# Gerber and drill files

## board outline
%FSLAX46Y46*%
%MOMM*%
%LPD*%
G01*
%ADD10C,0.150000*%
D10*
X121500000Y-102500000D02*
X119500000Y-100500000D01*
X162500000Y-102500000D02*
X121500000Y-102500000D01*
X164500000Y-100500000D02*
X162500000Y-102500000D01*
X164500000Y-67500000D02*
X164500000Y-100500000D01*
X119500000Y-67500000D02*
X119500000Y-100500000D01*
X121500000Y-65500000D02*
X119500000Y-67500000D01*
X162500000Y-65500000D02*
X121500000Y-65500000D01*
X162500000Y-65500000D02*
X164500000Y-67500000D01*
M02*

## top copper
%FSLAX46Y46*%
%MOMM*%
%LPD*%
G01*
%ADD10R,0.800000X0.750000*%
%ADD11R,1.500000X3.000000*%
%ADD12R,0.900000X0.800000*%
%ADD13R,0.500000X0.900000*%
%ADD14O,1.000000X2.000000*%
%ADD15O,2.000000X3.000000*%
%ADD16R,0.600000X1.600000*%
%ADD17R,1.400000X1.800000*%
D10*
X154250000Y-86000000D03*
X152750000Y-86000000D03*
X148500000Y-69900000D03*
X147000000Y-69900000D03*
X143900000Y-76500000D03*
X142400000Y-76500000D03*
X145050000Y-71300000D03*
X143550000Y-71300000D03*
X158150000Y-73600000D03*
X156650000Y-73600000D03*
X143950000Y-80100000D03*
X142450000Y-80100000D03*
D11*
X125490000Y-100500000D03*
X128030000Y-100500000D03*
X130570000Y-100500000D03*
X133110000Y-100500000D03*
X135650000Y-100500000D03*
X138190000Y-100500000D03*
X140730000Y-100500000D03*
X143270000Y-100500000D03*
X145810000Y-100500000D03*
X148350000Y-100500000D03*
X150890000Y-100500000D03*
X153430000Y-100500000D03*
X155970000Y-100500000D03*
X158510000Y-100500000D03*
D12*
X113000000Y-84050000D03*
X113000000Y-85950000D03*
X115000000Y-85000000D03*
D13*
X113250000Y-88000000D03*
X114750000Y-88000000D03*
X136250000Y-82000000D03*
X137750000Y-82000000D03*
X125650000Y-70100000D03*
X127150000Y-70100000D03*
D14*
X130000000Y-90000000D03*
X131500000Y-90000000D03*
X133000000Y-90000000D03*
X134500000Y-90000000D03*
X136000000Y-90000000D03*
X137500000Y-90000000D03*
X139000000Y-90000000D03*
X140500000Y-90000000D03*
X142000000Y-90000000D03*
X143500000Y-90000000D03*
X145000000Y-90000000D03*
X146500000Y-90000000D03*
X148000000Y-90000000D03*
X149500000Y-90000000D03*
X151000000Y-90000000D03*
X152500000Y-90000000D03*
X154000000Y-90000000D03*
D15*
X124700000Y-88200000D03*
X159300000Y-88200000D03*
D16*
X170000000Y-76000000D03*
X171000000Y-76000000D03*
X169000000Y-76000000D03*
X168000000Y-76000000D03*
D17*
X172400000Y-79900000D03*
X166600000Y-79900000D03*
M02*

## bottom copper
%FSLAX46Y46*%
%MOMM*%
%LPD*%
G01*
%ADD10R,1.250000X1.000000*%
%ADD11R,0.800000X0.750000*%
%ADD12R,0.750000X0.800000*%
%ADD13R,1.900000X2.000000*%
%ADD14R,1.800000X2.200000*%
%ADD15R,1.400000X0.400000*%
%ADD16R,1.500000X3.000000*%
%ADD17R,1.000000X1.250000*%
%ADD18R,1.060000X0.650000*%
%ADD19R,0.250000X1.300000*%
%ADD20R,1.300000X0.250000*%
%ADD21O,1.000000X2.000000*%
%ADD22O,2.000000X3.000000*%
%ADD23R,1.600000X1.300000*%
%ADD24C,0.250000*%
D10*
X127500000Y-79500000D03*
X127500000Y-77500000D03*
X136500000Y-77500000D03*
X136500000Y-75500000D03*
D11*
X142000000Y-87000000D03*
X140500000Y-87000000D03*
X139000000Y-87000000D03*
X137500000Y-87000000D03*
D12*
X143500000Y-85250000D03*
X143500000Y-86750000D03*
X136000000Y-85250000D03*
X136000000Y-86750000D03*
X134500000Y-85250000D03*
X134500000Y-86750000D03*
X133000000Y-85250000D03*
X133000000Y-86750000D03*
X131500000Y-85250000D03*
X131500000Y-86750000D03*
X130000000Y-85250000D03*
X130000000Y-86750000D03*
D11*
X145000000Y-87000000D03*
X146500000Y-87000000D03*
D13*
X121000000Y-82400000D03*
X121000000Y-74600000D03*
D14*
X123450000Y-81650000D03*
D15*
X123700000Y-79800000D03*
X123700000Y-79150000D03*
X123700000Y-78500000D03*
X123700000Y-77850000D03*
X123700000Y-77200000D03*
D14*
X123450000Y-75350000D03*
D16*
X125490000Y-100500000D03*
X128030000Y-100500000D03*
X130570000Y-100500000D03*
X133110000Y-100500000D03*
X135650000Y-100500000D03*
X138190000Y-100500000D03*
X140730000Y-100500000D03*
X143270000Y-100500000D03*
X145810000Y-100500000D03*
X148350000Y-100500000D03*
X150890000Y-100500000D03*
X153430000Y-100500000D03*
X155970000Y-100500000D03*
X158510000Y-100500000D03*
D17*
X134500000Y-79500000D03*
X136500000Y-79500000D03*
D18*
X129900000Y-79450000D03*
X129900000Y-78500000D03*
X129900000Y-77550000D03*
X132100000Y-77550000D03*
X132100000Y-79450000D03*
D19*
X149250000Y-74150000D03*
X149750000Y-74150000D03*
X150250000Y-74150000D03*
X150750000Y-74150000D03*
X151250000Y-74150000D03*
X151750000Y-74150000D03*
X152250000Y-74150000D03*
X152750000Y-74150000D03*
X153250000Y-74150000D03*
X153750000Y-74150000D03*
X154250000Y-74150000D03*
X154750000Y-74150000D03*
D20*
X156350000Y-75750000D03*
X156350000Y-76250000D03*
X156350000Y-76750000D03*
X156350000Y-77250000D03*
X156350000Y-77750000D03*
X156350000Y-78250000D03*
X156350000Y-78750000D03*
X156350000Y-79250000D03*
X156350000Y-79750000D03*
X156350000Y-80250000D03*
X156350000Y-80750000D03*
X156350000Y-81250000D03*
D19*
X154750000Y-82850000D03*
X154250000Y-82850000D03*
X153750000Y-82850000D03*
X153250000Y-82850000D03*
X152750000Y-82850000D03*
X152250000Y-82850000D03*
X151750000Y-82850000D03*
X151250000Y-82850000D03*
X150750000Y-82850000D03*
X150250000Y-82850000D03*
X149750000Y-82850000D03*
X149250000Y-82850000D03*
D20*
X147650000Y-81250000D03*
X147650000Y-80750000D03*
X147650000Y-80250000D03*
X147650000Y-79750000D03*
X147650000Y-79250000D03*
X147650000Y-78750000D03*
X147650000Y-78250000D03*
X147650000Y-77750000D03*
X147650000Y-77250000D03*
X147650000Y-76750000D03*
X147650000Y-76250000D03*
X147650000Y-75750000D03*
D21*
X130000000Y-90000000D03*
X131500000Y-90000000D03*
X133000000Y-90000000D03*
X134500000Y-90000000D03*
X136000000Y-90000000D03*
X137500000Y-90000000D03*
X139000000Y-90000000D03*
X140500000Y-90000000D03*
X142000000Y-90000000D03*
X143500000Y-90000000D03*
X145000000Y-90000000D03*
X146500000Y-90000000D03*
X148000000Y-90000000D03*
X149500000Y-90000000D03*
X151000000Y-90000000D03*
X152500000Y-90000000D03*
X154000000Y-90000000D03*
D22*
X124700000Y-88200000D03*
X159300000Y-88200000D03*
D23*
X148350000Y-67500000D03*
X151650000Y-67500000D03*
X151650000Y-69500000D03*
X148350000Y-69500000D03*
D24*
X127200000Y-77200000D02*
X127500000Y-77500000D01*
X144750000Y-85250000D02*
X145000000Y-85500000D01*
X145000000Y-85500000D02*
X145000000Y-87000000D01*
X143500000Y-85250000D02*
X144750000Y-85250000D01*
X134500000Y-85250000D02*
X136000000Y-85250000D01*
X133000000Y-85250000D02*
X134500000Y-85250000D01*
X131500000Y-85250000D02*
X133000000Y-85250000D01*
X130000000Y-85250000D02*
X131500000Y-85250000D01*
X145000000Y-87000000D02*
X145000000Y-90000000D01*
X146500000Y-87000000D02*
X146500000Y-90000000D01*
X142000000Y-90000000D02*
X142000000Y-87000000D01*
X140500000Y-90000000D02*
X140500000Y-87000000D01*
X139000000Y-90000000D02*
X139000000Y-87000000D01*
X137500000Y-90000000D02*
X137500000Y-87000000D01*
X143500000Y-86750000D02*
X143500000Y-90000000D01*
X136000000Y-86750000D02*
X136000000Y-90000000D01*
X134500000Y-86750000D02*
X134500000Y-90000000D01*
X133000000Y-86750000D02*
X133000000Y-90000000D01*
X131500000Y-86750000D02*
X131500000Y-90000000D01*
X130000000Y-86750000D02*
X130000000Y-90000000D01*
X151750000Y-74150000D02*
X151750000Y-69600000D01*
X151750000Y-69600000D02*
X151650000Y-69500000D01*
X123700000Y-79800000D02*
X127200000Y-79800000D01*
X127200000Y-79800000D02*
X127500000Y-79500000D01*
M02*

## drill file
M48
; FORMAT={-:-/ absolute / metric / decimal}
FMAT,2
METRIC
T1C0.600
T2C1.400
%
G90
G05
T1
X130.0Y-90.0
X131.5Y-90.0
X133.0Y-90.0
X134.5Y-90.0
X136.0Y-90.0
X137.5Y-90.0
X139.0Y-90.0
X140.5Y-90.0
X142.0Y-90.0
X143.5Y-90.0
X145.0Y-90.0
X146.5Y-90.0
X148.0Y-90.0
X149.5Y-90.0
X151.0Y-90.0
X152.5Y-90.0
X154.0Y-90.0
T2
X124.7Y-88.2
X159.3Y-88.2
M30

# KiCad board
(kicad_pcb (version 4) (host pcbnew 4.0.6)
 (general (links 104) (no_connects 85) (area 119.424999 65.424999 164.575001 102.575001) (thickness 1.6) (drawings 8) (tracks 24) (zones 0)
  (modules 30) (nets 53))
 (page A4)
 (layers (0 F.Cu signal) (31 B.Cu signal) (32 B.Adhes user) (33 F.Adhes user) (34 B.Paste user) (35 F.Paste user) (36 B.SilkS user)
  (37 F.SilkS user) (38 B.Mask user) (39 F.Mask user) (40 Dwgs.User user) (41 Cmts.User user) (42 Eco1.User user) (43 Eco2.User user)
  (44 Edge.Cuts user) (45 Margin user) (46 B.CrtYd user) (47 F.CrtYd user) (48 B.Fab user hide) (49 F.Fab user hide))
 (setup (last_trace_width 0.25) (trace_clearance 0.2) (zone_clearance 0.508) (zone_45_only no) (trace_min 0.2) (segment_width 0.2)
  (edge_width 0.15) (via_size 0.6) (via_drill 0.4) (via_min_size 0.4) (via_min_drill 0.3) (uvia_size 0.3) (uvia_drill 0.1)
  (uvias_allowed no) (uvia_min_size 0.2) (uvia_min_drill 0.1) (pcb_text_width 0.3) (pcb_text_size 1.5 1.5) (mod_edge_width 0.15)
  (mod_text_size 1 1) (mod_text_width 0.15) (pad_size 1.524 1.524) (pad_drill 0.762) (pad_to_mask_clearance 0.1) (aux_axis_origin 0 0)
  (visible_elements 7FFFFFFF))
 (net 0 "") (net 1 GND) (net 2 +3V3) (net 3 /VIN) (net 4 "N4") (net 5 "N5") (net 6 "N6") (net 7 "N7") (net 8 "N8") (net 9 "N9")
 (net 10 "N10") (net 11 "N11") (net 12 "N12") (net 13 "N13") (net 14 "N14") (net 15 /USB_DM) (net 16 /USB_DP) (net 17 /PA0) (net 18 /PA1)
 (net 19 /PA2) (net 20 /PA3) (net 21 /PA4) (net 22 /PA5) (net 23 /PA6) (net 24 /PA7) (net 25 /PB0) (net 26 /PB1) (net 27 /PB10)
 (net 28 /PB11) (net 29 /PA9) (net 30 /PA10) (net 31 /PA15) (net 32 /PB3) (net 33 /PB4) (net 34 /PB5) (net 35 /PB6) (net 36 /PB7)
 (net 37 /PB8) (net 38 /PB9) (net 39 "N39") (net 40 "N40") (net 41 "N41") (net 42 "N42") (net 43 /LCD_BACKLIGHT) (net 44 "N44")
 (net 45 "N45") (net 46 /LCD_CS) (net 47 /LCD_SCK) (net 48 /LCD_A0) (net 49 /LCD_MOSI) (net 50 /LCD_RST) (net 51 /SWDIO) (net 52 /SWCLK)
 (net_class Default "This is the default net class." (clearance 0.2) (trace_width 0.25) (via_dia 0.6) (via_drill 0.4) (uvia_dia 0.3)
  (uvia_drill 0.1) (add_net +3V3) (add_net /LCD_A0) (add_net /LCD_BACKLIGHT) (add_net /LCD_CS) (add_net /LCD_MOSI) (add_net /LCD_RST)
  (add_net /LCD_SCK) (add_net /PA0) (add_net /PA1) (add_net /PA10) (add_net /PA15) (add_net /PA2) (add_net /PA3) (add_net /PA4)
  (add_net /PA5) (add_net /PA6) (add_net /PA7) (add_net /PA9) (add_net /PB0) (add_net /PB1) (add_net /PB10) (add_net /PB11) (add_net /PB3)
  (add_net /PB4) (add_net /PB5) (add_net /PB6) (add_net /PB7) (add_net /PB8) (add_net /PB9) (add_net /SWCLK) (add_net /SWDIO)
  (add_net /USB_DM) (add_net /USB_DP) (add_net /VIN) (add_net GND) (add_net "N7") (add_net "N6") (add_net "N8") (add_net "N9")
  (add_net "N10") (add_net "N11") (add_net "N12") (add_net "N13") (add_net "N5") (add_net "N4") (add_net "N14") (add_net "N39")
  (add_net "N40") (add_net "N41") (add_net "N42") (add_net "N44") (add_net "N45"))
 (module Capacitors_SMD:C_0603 (layer F.Cu) (at 153.5 86)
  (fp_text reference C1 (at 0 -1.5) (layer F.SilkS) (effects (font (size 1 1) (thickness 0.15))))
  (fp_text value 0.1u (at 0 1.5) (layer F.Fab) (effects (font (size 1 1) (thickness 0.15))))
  (pad 2 smd rect (at 0.75 0) (size 0.8 0.75) (layers F.Cu F.Paste F.Mask) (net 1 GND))
  (pad 1 smd rect (at -0.75 0) (size 0.8 0.75) (layers F.Cu F.Paste F.Mask) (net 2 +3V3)))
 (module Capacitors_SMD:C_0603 (layer F.Cu) (at 147.75 69.9)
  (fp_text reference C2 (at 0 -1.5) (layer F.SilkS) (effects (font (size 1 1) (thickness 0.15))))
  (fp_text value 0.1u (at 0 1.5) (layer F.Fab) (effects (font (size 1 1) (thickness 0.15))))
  (pad 2 smd rect (at 0.75 0) (size 0.8 0.75) (layers F.Cu F.Paste F.Mask) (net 1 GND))
  (pad 1 smd rect (at -0.75 0) (size 0.8 0.75) (layers F.Cu F.Paste F.Mask) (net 2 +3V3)))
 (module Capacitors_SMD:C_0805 (layer B.Cu) (at 127.5 78.5 90)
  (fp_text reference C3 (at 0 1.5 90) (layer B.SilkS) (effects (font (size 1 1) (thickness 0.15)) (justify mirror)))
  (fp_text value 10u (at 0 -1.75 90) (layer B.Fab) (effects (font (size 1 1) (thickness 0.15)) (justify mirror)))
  (pad 1 smd rect (at -1 0 90) (size 1 1.25) (layers B.Cu B.Paste B.Mask) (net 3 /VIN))
  (pad 2 smd rect (at 1 0 90) (size 1 1.25) (layers B.Cu B.Paste B.Mask) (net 1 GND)))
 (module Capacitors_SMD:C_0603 (layer F.Cu) (at 143.15 76.5)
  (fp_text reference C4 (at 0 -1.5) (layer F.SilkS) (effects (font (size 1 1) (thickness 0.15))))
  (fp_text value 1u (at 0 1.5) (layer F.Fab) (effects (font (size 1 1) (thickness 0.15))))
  (pad 2 smd rect (at 0.75 0) (size 0.8 0.75) (layers F.Cu F.Paste F.Mask) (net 2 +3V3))
  (pad 1 smd rect (at -0.75 0) (size 0.8 0.75) (layers F.Cu F.Paste F.Mask) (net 1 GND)))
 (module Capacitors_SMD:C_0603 (layer F.Cu) (at 144.3 71.3)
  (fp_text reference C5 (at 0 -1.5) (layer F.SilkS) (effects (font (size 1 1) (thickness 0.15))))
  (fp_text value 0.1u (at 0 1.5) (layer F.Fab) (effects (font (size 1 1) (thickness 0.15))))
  (pad 2 smd rect (at 0.75 0) (size 0.8 0.75) (layers F.Cu F.Paste F.Mask) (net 1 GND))
  (pad 1 smd rect (at -0.75 0) (size 0.8 0.75) (layers F.Cu F.Paste F.Mask) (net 2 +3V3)))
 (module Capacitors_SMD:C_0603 (layer F.Cu) (at 157.4 73.6)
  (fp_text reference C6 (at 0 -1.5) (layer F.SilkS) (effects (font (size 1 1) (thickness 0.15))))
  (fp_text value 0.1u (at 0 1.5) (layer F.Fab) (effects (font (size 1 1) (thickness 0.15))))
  (pad 2 smd rect (at 0.75 0) (size 0.8 0.75) (layers F.Cu F.Paste F.Mask) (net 1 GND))
  (pad 1 smd rect (at -0.75 0) (size 0.8 0.75) (layers F.Cu F.Paste F.Mask) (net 2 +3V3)))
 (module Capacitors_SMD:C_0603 (layer F.Cu) (at 143.2 80.1)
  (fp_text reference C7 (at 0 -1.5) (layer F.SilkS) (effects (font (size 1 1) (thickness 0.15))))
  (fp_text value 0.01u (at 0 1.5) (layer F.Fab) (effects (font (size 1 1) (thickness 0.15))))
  (pad 2 smd rect (at 0.75 0) (size 0.8 0.75) (layers F.Cu F.Paste F.Mask) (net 2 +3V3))
  (pad 1 smd rect (at -0.75 0) (size 0.8 0.75) (layers F.Cu F.Paste F.Mask) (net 1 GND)))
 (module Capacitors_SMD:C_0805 (layer B.Cu) (at 136.5 76.5 90)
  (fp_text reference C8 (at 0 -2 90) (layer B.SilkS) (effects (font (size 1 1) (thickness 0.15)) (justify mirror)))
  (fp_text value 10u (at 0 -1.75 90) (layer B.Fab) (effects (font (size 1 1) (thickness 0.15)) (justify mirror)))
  (pad 1 smd rect (at -1 0 90) (size 1 1.25) (layers B.Cu B.Paste B.Mask) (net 2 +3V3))
  (pad 2 smd rect (at 1 0 90) (size 1 1.25) (layers B.Cu B.Paste B.Mask) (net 1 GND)))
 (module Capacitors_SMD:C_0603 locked (layer B.Cu) (at 141.25 87)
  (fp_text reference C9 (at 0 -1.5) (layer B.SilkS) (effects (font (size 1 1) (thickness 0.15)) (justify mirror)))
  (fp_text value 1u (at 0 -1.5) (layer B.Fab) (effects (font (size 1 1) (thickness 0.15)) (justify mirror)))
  (pad 2 smd rect (at 0.75 0) (size 0.8 0.75) (layers B.Cu B.Paste B.Mask) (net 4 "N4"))
  (pad 1 smd rect (at -0.75 0) (size 0.8 0.75) (layers B.Cu B.Paste B.Mask) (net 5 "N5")))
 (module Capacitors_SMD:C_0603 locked (layer B.Cu) (at 138.25 87)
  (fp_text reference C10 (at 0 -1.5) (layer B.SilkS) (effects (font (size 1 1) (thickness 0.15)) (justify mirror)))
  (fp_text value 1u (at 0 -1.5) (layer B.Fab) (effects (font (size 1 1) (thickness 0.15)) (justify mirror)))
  (pad 2 smd rect (at 0.75 0) (size 0.8 0.75) (layers B.Cu B.Paste B.Mask) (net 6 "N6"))
  (pad 1 smd rect (at -0.75 0) (size 0.8 0.75) (layers B.Cu B.Paste B.Mask) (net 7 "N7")))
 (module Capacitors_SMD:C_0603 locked (layer B.Cu) (at 143.5 86 90)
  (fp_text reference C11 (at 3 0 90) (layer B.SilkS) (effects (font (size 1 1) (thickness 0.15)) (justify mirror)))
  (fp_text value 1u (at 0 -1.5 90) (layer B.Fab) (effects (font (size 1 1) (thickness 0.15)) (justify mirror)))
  (pad 2 smd rect (at 0.75 0 90) (size 0.8 0.75) (layers B.Cu B.Paste B.Mask) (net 1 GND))
  (pad 1 smd rect (at -0.75 0 90) (size 0.8 0.75) (layers B.Cu B.Paste B.Mask) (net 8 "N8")))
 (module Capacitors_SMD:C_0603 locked (layer B.Cu) (at 136 86 90)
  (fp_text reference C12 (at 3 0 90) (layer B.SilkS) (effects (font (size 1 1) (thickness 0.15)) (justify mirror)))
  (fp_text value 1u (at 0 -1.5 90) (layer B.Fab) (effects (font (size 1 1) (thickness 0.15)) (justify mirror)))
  (pad 2 smd rect (at 0.75 0 90) (size 0.8 0.75) (layers B.Cu B.Paste B.Mask) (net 1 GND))
  (pad 1 smd rect (at -0.75 0 90) (size 0.8 0.75) (layers B.Cu B.Paste B.Mask) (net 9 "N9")))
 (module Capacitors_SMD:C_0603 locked (layer B.Cu) (at 134.5 86 90)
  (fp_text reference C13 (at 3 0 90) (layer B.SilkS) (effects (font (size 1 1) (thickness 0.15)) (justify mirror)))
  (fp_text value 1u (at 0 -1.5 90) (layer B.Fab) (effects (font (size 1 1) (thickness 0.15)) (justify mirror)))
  (pad 2 smd rect (at 0.75 0 90) (size 0.8 0.75) (layers B.Cu B.Paste B.Mask) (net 1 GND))
  (pad 1 smd rect (at -0.75 0 90) (size 0.8 0.75) (layers B.Cu B.Paste B.Mask) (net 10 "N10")))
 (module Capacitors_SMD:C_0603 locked (layer B.Cu) (at 133 86 90)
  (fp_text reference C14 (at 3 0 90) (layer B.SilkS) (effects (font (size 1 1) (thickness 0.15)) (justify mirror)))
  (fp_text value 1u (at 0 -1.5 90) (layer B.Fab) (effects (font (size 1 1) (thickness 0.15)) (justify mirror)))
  (pad 2 smd rect (at 0.75 0 90) (size 0.8 0.75) (layers B.Cu B.Paste B.Mask) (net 1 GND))
  (pad 1 smd rect (at -0.75 0 90) (size 0.8 0.75) (layers B.Cu B.Paste B.Mask) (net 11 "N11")))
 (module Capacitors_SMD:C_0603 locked (layer B.Cu) (at 131.5 86 90)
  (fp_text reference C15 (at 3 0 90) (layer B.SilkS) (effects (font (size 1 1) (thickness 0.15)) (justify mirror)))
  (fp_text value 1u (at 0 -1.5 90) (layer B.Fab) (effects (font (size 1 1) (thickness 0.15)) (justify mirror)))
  (pad 2 smd rect (at 0.75 0 90) (size 0.8 0.75) (layers B.Cu B.Paste B.Mask) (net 1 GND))
  (pad 1 smd rect (at -0.75 0 90) (size 0.8 0.75) (layers B.Cu B.Paste B.Mask) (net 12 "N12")))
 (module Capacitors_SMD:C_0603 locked (layer B.Cu) (at 130 86 90)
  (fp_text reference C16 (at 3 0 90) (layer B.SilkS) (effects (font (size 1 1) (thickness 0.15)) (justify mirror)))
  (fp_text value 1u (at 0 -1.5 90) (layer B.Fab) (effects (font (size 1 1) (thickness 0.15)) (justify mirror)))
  (pad 2 smd rect (at 0.75 0 90) (size 0.8 0.75) (layers B.Cu B.Paste B.Mask) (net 1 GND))
  (pad 1 smd rect (at -0.75 0 90) (size 0.8 0.75) (layers B.Cu B.Paste B.Mask) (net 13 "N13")))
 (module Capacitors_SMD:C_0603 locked (layer B.Cu) (at 145.75 87 180)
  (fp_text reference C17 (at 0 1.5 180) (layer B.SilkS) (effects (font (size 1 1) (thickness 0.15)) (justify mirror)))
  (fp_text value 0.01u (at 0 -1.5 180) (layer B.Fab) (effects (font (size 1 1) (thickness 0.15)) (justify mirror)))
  (pad 2 smd rect (at 0.75 0 180) (size 0.8 0.75) (layers B.Cu B.Paste B.Mask) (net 1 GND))
  (pad 1 smd rect (at -0.75 0 180) (size 0.8 0.75) (layers B.Cu B.Paste B.Mask) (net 2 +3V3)))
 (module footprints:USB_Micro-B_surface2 (layer B.Cu) (at 121 78.5 90) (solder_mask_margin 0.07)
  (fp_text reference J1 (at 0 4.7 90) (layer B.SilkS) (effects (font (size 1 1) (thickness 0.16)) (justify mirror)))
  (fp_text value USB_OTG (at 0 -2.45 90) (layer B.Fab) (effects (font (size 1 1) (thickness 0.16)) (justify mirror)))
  (pad 6 smd rect (at -3.9 0 90) (size 2 1.9) (layers B.Cu B.Mask) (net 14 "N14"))
  (pad 6 smd rect (at 3.9 0 90) (size 2 1.9) (layers B.Cu B.Mask) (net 14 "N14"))
  (pad 6 smd rect (at -3.15 2.45 90) (size 2.2 1.8) (layers B.Cu B.Mask) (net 14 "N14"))
  (pad 1 smd rect (at -1.3 2.7) (size 1.4 0.4) (layers B.Cu B.Mask) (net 3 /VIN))
  (pad 2 smd rect (at -0.65 2.7) (size 1.4 0.4) (layers B.Cu B.Mask) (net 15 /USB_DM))
  (pad 3 smd rect (at 0 2.7) (size 1.4 0.4) (layers B.Cu B.Mask) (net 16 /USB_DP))
  (pad 4 smd rect (at 0.65 2.7) (size 1.4 0.4) (layers B.Cu B.Mask))
  (pad 5 smd rect (at 1.3 2.7) (size 1.4 0.4) (layers B.Cu B.Mask) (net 1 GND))
  (pad 6 smd rect (at 3.15 2.45 90) (size 2.2 1.8) (layers B.Cu B.Mask) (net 14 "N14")))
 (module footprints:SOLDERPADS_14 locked (layer B.Cu) (at 142 100.5)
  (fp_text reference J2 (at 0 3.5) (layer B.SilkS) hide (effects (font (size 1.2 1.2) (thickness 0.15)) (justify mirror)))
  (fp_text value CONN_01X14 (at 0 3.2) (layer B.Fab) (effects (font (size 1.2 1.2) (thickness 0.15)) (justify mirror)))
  (pad 1 smd rect (at -16.51 0) (size 1.5 3) (layers B.Cu B.Paste B.Mask) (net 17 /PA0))
  (pad 2 smd rect (at -13.97 0) (size 1.5 3) (layers B.Cu B.Paste B.Mask) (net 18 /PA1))
  (pad 3 smd rect (at -11.43 0) (size 1.5 3) (layers B.Cu B.Paste B.Mask) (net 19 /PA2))
  (pad 4 smd rect (at -8.89 0) (size 1.5 3) (layers B.Cu B.Paste B.Mask) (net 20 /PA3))
  (pad 5 smd rect (at -6.35 0) (size 1.5 3) (layers B.Cu B.Paste B.Mask) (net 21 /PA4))
  (pad 6 smd rect (at -3.81 0) (size 1.5 3) (layers B.Cu B.Paste B.Mask) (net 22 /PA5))
  (pad 7 smd rect (at -1.27 0) (size 1.5 3) (layers B.Cu B.Paste B.Mask) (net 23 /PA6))
  (pad 8 smd rect (at 1.27 0) (size 1.5 3) (layers B.Cu B.Paste B.Mask) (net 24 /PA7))
  (pad 9 smd rect (at 3.81 0) (size 1.5 3) (layers B.Cu B.Paste B.Mask) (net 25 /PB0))
  (pad 10 smd rect (at 6.35 0) (size 1.5 3) (layers B.Cu B.Paste B.Mask) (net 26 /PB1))
  (pad 11 smd rect (at 8.89 0) (size 1.5 3) (layers B.Cu B.Paste B.Mask) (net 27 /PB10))
  (pad 12 smd rect (at 11.43 0) (size 1.5 3) (layers B.Cu B.Paste B.Mask) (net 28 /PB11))
  (pad 13 smd rect (at 13.97 0) (size 1.5 3) (layers B.Cu B.Paste B.Mask) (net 2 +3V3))
  (pad 14 smd rect (at 16.51 0) (size 1.5 3) (layers B.Cu B.Paste B.Mask) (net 1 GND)))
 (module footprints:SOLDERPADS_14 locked (layer F.Cu) (at 142 100.5)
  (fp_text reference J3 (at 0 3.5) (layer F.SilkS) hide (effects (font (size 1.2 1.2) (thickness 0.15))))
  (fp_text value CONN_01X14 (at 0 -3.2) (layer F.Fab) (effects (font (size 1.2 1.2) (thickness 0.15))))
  (pad 1 smd rect (at -16.51 0) (size 1.5 3) (layers F.Cu F.Paste F.Mask) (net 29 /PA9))
  (pad 2 smd rect (at -13.97 0) (size 1.5 3) (layers F.Cu F.Paste F.Mask) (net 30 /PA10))
  (pad 3 smd rect (at -11.43 0) (size 1.5 3) (layers F.Cu F.Paste F.Mask) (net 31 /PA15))
  (pad 4 smd rect (at -8.89 0) (size 1.5 3) (layers F.Cu F.Paste F.Mask) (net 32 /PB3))
  (pad 5 smd rect (at -6.35 0) (size 1.5 3) (layers F.Cu F.Paste F.Mask) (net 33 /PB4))
  (pad 6 smd rect (at -3.81 0) (size 1.5 3) (layers F.Cu F.Paste F.Mask) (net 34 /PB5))
  (pad 7 smd rect (at -1.27 0) (size 1.5 3) (layers F.Cu F.Paste F.Mask) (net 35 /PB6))
  (pad 8 smd rect (at 1.27 0) (size 1.5 3) (layers F.Cu F.Paste F.Mask) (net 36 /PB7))
  (pad 9 smd rect (at 3.81 0) (size 1.5 3) (layers F.Cu F.Paste F.Mask) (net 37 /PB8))
  (pad 10 smd rect (at 6.35 0) (size 1.5 3) (layers F.Cu F.Paste F.Mask) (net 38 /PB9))
  (pad 11 smd rect (at 8.89 0) (size 1.5 3) (layers F.Cu F.Paste F.Mask) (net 27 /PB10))
  (pad 12 smd rect (at 11.43 0) (size 1.5 3) (layers F.Cu F.Paste F.Mask) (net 28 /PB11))
  (pad 13 smd rect (at 13.97 0) (size 1.5 3) (layers F.Cu F.Paste F.Mask) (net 2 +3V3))
  (pad 14 smd rect (at 16.51 0) (size 1.5 3) (layers F.Cu F.Paste F.Mask) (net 1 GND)))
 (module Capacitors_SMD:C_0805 (layer B.Cu) (at 135.5 79.5)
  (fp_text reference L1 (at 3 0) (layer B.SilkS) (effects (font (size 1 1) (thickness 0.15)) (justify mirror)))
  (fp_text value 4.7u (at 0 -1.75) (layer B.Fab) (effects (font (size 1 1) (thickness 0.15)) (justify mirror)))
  (pad 1 smd rect (at -1 0) (size 1 1.25) (layers B.Cu B.Paste B.Mask) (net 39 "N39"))
  (pad 2 smd rect (at 1 0) (size 1 1.25) (layers B.Cu B.Paste B.Mask) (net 2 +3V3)))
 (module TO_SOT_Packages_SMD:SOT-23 (layer F.Cu) (at 114 85)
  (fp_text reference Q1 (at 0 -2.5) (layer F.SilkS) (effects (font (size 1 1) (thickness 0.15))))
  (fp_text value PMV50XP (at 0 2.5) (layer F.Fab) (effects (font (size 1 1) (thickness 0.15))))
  (pad 1 smd rect (at -1 -0.95) (size 0.9 0.8) (layers F.Cu F.Paste F.Mask) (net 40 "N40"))
  (pad 2 smd rect (at -1 0.95) (size 0.9 0.8) (layers F.Cu F.Paste F.Mask) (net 2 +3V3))
  (pad 3 smd rect (at 1 0) (size 0.9 0.8) (layers F.Cu F.Paste F.Mask) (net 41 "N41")))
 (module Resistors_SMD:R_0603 (layer F.Cu) (at 114 88)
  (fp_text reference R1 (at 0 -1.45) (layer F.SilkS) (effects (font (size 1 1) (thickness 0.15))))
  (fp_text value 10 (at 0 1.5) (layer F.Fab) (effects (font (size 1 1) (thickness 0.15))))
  (pad 1 smd rect (at -0.75 0) (size 0.5 0.9) (layers F.Cu F.Paste F.Mask) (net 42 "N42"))
  (pad 2 smd rect (at 0.75 0) (size 0.5 0.9) (layers F.Cu F.Paste F.Mask) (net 41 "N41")))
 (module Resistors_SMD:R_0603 (layer F.Cu) (at 137 82)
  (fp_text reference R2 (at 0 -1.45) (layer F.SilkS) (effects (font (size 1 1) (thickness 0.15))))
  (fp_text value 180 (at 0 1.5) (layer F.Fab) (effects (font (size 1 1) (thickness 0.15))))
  (pad 1 smd rect (at -0.75 0) (size 0.5 0.9) (layers F.Cu F.Paste F.Mask) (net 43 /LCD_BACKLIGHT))
  (pad 2 smd rect (at 0.75 0) (size 0.5 0.9) (layers F.Cu F.Paste F.Mask) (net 40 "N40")))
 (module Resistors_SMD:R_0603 (layer F.Cu) (at 126.4 70.1)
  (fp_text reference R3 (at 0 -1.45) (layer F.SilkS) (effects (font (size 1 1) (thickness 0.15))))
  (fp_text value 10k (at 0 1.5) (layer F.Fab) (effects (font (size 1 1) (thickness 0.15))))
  (pad 1 smd rect (at -0.75 0) (size 0.5 0.9) (layers F.Cu F.Paste F.Mask) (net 2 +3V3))
  (pad 2 smd rect (at 0.75 0) (size 0.5 0.9) (layers F.Cu F.Paste F.Mask) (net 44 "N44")))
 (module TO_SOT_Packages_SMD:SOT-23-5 (layer B.Cu) (at 131 78.5)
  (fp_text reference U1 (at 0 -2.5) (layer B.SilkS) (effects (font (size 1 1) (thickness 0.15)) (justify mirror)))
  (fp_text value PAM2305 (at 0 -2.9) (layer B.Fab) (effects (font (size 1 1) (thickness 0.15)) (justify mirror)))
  (pad 1 smd rect (at -1.1 0.95) (size 1.06 0.65) (layers B.Cu B.Paste B.Mask) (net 3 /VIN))
  (pad 2 smd rect (at -1.1 0) (size 1.06 0.65) (layers B.Cu B.Paste B.Mask) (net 1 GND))
  (pad 3 smd rect (at -1.1 -0.95) (size 1.06 0.65) (layers B.Cu B.Paste B.Mask) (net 3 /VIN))
  (pad 4 smd rect (at 1.1 -0.95) (size 1.06 0.65) (layers B.Cu B.Paste B.Mask) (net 2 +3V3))
  (pad 5 smd rect (at 1.1 0.95) (size 1.06 0.65) (layers B.Cu B.Paste B.Mask) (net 39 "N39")))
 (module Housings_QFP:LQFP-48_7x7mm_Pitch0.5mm (layer B.Cu) (at 152 78.5 270)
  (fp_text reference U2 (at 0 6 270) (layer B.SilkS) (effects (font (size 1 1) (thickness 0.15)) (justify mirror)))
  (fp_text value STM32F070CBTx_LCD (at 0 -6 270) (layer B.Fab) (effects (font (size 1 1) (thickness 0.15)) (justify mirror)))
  (pad 1 smd rect (at -4.35 2.75 270) (size 1.3 0.25) (layers B.Cu B.Paste B.Mask) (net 2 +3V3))
  (pad 2 smd rect (at -4.35 2.25 270) (size 1.3 0.25) (layers B.Cu B.Paste B.Mask))
  (pad 3 smd rect (at -4.35 1.75 270) (size 1.3 0.25) (layers B.Cu B.Paste B.Mask))
  (pad 4 smd rect (at -4.35 1.25 270) (size 1.3 0.25) (layers B.Cu B.Paste B.Mask))
  (pad 5 smd rect (at -4.35 0.75 270) (size 1.3 0.25) (layers B.Cu B.Paste B.Mask))
  (pad 6 smd rect (at -4.35 0.25 270) (size 1.3 0.25) (layers B.Cu B.Paste B.Mask) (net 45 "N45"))
  (pad 7 smd rect (at -4.35 -0.25 270) (size 1.3 0.25) (layers B.Cu B.Paste B.Mask))
  (pad 8 smd rect (at -4.35 -0.75 270) (size 1.3 0.25) (layers B.Cu B.Paste B.Mask) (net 1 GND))
  (pad 9 smd rect (at -4.35 -1.25 270) (size 1.3 0.25) (layers B.Cu B.Paste B.Mask) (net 2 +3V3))
  (pad 10 smd rect (at -4.35 -1.75 270) (size 1.3 0.25) (layers B.Cu B.Paste B.Mask) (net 17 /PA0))
  (pad 11 smd rect (at -4.35 -2.25 270) (size 1.3 0.25) (layers B.Cu B.Paste B.Mask) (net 18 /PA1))
  (pad 12 smd rect (at -4.35 -2.75 270) (size 1.3 0.25) (layers B.Cu B.Paste B.Mask) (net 19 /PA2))
  (pad 13 smd rect (at -2.75 -4.35 180) (size 1.3 0.25) (layers B.Cu B.Paste B.Mask) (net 20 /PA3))
  (pad 14 smd rect (at -2.25 -4.35 180) (size 1.3 0.25) (layers B.Cu B.Paste B.Mask) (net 21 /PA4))
  (pad 15 smd rect (at -1.75 -4.35 180) (size 1.3 0.25) (layers B.Cu B.Paste B.Mask) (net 22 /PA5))
  (pad 16 smd rect (at -1.25 -4.35 180) (size 1.3 0.25) (layers B.Cu B.Paste B.Mask) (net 23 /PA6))
  (pad 17 smd rect (at -0.75 -4.35 180) (size 1.3 0.25) (layers B.Cu B.Paste B.Mask) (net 24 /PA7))
  (pad 18 smd rect (at -0.25 -4.35 180) (size 1.3 0.25) (layers B.Cu B.Paste B.Mask) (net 25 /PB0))
  (pad 19 smd rect (at 0.25 -4.35 180) (size 1.3 0.25) (layers B.Cu B.Paste B.Mask) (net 26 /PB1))
  (pad 20 smd rect (at 0.75 -4.35 180) (size 1.3 0.25) (layers B.Cu B.Paste B.Mask) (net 43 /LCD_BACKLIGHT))
  (pad 21 smd rect (at 1.25 -4.35 180) (size 1.3 0.25) (layers B.Cu B.Paste B.Mask) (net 27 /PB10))
  (pad 22 smd rect (at 1.75 -4.35 180) (size 1.3 0.25) (layers B.Cu B.Paste B.Mask) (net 28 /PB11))
  (pad 23 smd rect (at 2.25 -4.35 180) (size 1.3 0.25) (layers B.Cu B.Paste B.Mask) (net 1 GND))
  (pad 24 smd rect (at 2.75 -4.35 180) (size 1.3 0.25) (layers B.Cu B.Paste B.Mask) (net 2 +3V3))
  (pad 25 smd rect (at 4.35 -2.75 270) (size 1.3 0.25) (layers B.Cu B.Paste B.Mask) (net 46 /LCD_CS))
  (pad 26 smd rect (at 4.35 -2.25 270) (size 1.3 0.25) (layers B.Cu B.Paste B.Mask) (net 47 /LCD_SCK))
  (pad 27 smd rect (at 4.35 -1.75 270) (size 1.3 0.25) (layers B.Cu B.Paste B.Mask) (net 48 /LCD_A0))
  (pad 28 smd rect (at 4.35 -1.25 270) (size 1.3 0.25) (layers B.Cu B.Paste B.Mask) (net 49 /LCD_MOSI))
  (pad 29 smd rect (at 4.35 -0.75 270) (size 1.3 0.25) (layers B.Cu B.Paste B.Mask) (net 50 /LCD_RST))
  (pad 30 smd rect (at 4.35 -0.25 270) (size 1.3 0.25) (layers B.Cu B.Paste B.Mask) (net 29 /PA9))
  (pad 31 smd rect (at 4.35 0.25 270) (size 1.3 0.25) (layers B.Cu B.Paste B.Mask) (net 30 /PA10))
  (pad 32 smd rect (at 4.35 0.75 270) (size 1.3 0.25) (layers B.Cu B.Paste B.Mask) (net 15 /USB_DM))
  (pad 33 smd rect (at 4.35 1.25 270) (size 1.3 0.25) (layers B.Cu B.Paste B.Mask) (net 16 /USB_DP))
  (pad 34 smd rect (at 4.35 1.75 270) (size 1.3 0.25) (layers B.Cu B.Paste B.Mask) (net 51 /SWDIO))
  (pad 35 smd rect (at 4.35 2.25 270) (size 1.3 0.25) (layers B.Cu B.Paste B.Mask) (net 1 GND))
  (pad 36 smd rect (at 4.35 2.75 270) (size 1.3 0.25) (layers B.Cu B.Paste B.Mask) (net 2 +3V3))
  (pad 37 smd rect (at 2.75 4.35 180) (size 1.3 0.25) (layers B.Cu B.Paste B.Mask) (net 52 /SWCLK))
  (pad 38 smd rect (at 2.25 4.35 180) (size 1.3 0.25) (layers B.Cu B.Paste B.Mask) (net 31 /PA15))
  (pad 39 smd rect (at 1.75 4.35 180) (size 1.3 0.25) (layers B.Cu B.Paste B.Mask) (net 32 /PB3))
  (pad 40 smd rect (at 1.25 4.35 180) (size 1.3 0.25) (layers B.Cu B.Paste B.Mask) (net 33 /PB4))
  (pad 41 smd rect (at 0.75 4.35 180) (size 1.3 0.25) (layers B.Cu B.Paste B.Mask) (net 34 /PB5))
  (pad 42 smd rect (at 0.25 4.35 180) (size 1.3 0.25) (layers B.Cu B.Paste B.Mask) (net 35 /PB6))
  (pad 43 smd rect (at -0.25 4.35 180) (size 1.3 0.25) (layers B.Cu B.Paste B.Mask) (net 36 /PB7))
  (pad 44 smd rect (at -0.75 4.35 180) (size 1.3 0.25) (layers B.Cu B.Paste B.Mask) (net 1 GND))
  (pad 45 smd rect (at -1.25 4.35 180) (size 1.3 0.25) (layers B.Cu B.Paste B.Mask) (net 37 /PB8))
  (pad 46 smd rect (at -1.75 4.35 180) (size 1.3 0.25) (layers B.Cu B.Paste B.Mask) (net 38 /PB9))
  (pad 47 smd rect (at -2.25 4.35 180) (size 1.3 0.25) (layers B.Cu B.Paste B.Mask) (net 1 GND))
  (pad 48 smd rect (at -2.75 4.35 180) (size 1.3 0.25) (layers B.Cu B.Paste B.Mask) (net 2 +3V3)))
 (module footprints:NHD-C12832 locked (layer F.Cu) (at 142 90)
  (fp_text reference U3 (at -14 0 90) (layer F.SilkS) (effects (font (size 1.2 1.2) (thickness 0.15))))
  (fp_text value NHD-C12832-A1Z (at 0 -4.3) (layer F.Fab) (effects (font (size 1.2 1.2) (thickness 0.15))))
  (pad 1 thru_hole oval (at -12 0) (size 1 2) (drill 0.6) (layers *.Cu *.Mask) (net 13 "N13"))
  (pad 2 thru_hole oval (at -10.5 0) (size 1 2) (drill 0.6) (layers *.Cu *.Mask) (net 12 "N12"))
  (pad 3 thru_hole oval (at -9 0) (size 1 2) (drill 0.6) (layers *.Cu *.Mask) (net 11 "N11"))
  (pad 4 thru_hole oval (at -7.5 0) (size 1 2) (drill 0.6) (layers *.Cu *.Mask) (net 10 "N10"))
  (pad 5 thru_hole oval (at -6 0) (size 1 2) (drill 0.6) (layers *.Cu *.Mask) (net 9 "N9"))
  (pad 6 thru_hole oval (at -4.5 0) (size 1 2) (drill 0.6) (layers *.Cu *.Mask) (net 7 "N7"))
  (pad 7 thru_hole oval (at -3 0) (size 1 2) (drill 0.6) (layers *.Cu *.Mask) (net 6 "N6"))
  (pad 8 thru_hole oval (at -1.5 0) (size 1 2) (drill 0.6) (layers *.Cu *.Mask) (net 5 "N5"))
  (pad 9 thru_hole oval (at 0 0) (size 1 2) (drill 0.6) (layers *.Cu *.Mask) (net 4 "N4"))
  (pad 10 thru_hole oval (at 1.5 0) (size 1 2) (drill 0.6) (layers *.Cu *.Mask) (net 8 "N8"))
  (pad 11 thru_hole oval (at 3 0) (size 1 2) (drill 0.6) (layers *.Cu *.Mask) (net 1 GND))
  (pad 12 thru_hole oval (at 4.5 0) (size 1 2) (drill 0.6) (layers *.Cu *.Mask) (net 2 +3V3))
  (pad 13 thru_hole oval (at 6 0) (size 1 2) (drill 0.6) (layers *.Cu *.Mask) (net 49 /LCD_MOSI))
  (pad 14 thru_hole oval (at 7.5 0) (size 1 2) (drill 0.6) (layers *.Cu *.Mask) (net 47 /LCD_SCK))
  (pad 15 thru_hole oval (at 9 0) (size 1 2) (drill 0.6) (layers *.Cu *.Mask) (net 48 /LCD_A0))
  (pad 16 thru_hole oval (at 10.5 0) (size 1 2) (drill 0.6) (layers *.Cu *.Mask) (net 50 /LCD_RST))
  (pad 17 thru_hole oval (at 12 0) (size 1 2) (drill 0.6) (layers *.Cu *.Mask) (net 46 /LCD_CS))
  (pad 18 thru_hole oval (at -17.3 -1.8) (size 2 3) (drill 1.4) (layers *.Cu *.Mask) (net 42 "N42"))
  (pad 19 thru_hole oval (at 17.3 -1.8) (size 2 3) (drill 1.4) (layers *.Cu *.Mask) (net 1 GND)))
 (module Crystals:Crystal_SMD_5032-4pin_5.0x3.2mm (layer B.Cu) (at 150 68.5)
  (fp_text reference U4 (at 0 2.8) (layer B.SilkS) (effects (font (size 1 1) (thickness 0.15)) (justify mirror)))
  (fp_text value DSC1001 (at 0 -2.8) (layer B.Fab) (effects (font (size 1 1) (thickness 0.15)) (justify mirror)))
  (pad 1 smd rect (at -1.65 -1) (size 1.6 1.3) (layers B.Cu B.Paste B.Mask) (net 44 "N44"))
  (pad 2 smd rect (at 1.65 -1) (size 1.6 1.3) (layers B.Cu B.Paste B.Mask) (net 1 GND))
  (pad 3 smd rect (at 1.65 1) (size 1.6 1.3) (layers B.Cu B.Paste B.Mask) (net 45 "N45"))
  (pad 4 smd rect (at -1.65 1) (size 1.6 1.3) (layers B.Cu B.Paste B.Mask) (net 2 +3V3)))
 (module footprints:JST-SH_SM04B (layer F.Cu) (at 169.5 75.2)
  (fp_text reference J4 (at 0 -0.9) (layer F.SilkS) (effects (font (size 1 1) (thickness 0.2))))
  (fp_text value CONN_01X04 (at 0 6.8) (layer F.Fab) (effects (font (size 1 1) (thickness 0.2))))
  (pad 3 smd rect (at 0.5 0.8) (size 0.6 1.6) (layers F.Cu F.Paste F.Mask) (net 2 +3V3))
  (pad 4 smd rect (at 1.5 0.8) (size 0.6 1.6) (layers F.Cu F.Paste F.Mask) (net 1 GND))
  (pad 2 smd rect (at -0.5 0.8) (size 0.6 1.6) (layers F.Cu F.Paste F.Mask) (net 52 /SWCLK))
  (pad 1 smd rect (at -1.5 0.8) (size 0.6 1.6) (layers F.Cu F.Paste F.Mask) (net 51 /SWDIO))
  (pad "" smd rect (at 2.9 4.7) (size 1.4 1.8) (layers F.Cu F.Paste F.Mask))
  (pad "" smd rect (at -2.9 4.7) (size 1.4 1.8) (layers F.Cu F.Paste F.Mask)))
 (gr_line (start 121.5 102.5) (end 119.5 100.5) (layer Edge.Cuts) (width 0.15))
 (gr_line (start 162.5 102.5) (end 121.5 102.5) (layer Edge.Cuts) (width 0.15))
 (gr_line (start 164.5 100.5) (end 162.5 102.5) (layer Edge.Cuts) (width 0.15))
 (gr_line (start 164.5 67.5) (end 164.5 100.5) (layer Edge.Cuts) (width 0.15))
 (gr_line (start 119.5 67.5) (end 119.5 100.5) (layer Edge.Cuts) (width 0.15))
 (gr_line (start 121.5 65.5) (end 119.5 67.5) (layer Edge.Cuts) (width 0.15))
 (gr_line (start 162.5 65.5) (end 121.5 65.5) (layer Edge.Cuts) (width 0.15))
 (gr_line (start 162.5 65.5) (end 164.5 67.5) (layer Edge.Cuts) (width 0.15))
 (segment (start 127.2 77.2) (end 127.5 77.5) (width 0.25) (layer B.Cu) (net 1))
 (segment (start 144.75 85.25) (end 145 85.5) (width 0.25) (layer B.Cu) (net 1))
 (segment (start 145 85.5) (end 145 87) (width 0.25) (layer B.Cu) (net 1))
 (segment (start 143.5 85.25) (end 144.75 85.25) (width 0.25) (layer B.Cu) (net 1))
 (segment (start 134.5 85.25) (end 136 85.25) (width 0.25) (layer B.Cu) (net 1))
 (segment (start 133 85.25) (end 134.5 85.25) (width 0.25) (layer B.Cu) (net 1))
 (segment (start 131.5 85.25) (end 133 85.25) (width 0.25) (layer B.Cu) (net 1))
 (segment (start 130 85.25) (end 131.5 85.25) (width 0.25) (layer B.Cu) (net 1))
 (segment (start 145 87) (end 145 90) (width 0.25) (layer B.Cu) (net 1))
 (segment (start 146.5 87) (end 146.5 90) (width 0.25) (layer B.Cu) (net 2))
 (segment (start 142 90) (end 142 87) (width 0.25) (layer B.Cu) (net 4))
 (segment (start 140.5 90) (end 140.5 87) (width 0.25) (layer B.Cu) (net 5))
 (segment (start 139 90) (end 139 87) (width 0.25) (layer B.Cu) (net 6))
 (segment (start 137.5 90) (end 137.5 87) (width 0.25) (layer B.Cu) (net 7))
 (segment (start 143.5 86.75) (end 143.5 90) (width 0.25) (layer B.Cu) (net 8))
 (segment (start 136 86.75) (end 136 90) (width 0.25) (layer B.Cu) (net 9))
 (segment (start 134.5 86.75) (end 134.5 90) (width 0.25) (layer B.Cu) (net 10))
 (segment (start 133 86.75) (end 133 90) (width 0.25) (layer B.Cu) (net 11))
 (segment (start 131.5 86.75) (end 131.5 90) (width 0.25) (layer B.Cu) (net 12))
 (segment (start 130 86.75) (end 130 90) (width 0.25) (layer B.Cu) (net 13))
 (segment (start 151.75 74.15) (end 151.75 69.6) (width 0.25) (layer B.Cu) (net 45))
 (segment (start 151.75 69.6) (end 151.65 69.5) (width 0.25) (layer B.Cu) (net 45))
 (segment (start 123.7 79.8) (end 127.2 79.8) (width 0.25) (layer B.Cu) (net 3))
 (segment (start 127.2 79.8) (end 127.5 79.5) (width 0.25) (layer B.Cu) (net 3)))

